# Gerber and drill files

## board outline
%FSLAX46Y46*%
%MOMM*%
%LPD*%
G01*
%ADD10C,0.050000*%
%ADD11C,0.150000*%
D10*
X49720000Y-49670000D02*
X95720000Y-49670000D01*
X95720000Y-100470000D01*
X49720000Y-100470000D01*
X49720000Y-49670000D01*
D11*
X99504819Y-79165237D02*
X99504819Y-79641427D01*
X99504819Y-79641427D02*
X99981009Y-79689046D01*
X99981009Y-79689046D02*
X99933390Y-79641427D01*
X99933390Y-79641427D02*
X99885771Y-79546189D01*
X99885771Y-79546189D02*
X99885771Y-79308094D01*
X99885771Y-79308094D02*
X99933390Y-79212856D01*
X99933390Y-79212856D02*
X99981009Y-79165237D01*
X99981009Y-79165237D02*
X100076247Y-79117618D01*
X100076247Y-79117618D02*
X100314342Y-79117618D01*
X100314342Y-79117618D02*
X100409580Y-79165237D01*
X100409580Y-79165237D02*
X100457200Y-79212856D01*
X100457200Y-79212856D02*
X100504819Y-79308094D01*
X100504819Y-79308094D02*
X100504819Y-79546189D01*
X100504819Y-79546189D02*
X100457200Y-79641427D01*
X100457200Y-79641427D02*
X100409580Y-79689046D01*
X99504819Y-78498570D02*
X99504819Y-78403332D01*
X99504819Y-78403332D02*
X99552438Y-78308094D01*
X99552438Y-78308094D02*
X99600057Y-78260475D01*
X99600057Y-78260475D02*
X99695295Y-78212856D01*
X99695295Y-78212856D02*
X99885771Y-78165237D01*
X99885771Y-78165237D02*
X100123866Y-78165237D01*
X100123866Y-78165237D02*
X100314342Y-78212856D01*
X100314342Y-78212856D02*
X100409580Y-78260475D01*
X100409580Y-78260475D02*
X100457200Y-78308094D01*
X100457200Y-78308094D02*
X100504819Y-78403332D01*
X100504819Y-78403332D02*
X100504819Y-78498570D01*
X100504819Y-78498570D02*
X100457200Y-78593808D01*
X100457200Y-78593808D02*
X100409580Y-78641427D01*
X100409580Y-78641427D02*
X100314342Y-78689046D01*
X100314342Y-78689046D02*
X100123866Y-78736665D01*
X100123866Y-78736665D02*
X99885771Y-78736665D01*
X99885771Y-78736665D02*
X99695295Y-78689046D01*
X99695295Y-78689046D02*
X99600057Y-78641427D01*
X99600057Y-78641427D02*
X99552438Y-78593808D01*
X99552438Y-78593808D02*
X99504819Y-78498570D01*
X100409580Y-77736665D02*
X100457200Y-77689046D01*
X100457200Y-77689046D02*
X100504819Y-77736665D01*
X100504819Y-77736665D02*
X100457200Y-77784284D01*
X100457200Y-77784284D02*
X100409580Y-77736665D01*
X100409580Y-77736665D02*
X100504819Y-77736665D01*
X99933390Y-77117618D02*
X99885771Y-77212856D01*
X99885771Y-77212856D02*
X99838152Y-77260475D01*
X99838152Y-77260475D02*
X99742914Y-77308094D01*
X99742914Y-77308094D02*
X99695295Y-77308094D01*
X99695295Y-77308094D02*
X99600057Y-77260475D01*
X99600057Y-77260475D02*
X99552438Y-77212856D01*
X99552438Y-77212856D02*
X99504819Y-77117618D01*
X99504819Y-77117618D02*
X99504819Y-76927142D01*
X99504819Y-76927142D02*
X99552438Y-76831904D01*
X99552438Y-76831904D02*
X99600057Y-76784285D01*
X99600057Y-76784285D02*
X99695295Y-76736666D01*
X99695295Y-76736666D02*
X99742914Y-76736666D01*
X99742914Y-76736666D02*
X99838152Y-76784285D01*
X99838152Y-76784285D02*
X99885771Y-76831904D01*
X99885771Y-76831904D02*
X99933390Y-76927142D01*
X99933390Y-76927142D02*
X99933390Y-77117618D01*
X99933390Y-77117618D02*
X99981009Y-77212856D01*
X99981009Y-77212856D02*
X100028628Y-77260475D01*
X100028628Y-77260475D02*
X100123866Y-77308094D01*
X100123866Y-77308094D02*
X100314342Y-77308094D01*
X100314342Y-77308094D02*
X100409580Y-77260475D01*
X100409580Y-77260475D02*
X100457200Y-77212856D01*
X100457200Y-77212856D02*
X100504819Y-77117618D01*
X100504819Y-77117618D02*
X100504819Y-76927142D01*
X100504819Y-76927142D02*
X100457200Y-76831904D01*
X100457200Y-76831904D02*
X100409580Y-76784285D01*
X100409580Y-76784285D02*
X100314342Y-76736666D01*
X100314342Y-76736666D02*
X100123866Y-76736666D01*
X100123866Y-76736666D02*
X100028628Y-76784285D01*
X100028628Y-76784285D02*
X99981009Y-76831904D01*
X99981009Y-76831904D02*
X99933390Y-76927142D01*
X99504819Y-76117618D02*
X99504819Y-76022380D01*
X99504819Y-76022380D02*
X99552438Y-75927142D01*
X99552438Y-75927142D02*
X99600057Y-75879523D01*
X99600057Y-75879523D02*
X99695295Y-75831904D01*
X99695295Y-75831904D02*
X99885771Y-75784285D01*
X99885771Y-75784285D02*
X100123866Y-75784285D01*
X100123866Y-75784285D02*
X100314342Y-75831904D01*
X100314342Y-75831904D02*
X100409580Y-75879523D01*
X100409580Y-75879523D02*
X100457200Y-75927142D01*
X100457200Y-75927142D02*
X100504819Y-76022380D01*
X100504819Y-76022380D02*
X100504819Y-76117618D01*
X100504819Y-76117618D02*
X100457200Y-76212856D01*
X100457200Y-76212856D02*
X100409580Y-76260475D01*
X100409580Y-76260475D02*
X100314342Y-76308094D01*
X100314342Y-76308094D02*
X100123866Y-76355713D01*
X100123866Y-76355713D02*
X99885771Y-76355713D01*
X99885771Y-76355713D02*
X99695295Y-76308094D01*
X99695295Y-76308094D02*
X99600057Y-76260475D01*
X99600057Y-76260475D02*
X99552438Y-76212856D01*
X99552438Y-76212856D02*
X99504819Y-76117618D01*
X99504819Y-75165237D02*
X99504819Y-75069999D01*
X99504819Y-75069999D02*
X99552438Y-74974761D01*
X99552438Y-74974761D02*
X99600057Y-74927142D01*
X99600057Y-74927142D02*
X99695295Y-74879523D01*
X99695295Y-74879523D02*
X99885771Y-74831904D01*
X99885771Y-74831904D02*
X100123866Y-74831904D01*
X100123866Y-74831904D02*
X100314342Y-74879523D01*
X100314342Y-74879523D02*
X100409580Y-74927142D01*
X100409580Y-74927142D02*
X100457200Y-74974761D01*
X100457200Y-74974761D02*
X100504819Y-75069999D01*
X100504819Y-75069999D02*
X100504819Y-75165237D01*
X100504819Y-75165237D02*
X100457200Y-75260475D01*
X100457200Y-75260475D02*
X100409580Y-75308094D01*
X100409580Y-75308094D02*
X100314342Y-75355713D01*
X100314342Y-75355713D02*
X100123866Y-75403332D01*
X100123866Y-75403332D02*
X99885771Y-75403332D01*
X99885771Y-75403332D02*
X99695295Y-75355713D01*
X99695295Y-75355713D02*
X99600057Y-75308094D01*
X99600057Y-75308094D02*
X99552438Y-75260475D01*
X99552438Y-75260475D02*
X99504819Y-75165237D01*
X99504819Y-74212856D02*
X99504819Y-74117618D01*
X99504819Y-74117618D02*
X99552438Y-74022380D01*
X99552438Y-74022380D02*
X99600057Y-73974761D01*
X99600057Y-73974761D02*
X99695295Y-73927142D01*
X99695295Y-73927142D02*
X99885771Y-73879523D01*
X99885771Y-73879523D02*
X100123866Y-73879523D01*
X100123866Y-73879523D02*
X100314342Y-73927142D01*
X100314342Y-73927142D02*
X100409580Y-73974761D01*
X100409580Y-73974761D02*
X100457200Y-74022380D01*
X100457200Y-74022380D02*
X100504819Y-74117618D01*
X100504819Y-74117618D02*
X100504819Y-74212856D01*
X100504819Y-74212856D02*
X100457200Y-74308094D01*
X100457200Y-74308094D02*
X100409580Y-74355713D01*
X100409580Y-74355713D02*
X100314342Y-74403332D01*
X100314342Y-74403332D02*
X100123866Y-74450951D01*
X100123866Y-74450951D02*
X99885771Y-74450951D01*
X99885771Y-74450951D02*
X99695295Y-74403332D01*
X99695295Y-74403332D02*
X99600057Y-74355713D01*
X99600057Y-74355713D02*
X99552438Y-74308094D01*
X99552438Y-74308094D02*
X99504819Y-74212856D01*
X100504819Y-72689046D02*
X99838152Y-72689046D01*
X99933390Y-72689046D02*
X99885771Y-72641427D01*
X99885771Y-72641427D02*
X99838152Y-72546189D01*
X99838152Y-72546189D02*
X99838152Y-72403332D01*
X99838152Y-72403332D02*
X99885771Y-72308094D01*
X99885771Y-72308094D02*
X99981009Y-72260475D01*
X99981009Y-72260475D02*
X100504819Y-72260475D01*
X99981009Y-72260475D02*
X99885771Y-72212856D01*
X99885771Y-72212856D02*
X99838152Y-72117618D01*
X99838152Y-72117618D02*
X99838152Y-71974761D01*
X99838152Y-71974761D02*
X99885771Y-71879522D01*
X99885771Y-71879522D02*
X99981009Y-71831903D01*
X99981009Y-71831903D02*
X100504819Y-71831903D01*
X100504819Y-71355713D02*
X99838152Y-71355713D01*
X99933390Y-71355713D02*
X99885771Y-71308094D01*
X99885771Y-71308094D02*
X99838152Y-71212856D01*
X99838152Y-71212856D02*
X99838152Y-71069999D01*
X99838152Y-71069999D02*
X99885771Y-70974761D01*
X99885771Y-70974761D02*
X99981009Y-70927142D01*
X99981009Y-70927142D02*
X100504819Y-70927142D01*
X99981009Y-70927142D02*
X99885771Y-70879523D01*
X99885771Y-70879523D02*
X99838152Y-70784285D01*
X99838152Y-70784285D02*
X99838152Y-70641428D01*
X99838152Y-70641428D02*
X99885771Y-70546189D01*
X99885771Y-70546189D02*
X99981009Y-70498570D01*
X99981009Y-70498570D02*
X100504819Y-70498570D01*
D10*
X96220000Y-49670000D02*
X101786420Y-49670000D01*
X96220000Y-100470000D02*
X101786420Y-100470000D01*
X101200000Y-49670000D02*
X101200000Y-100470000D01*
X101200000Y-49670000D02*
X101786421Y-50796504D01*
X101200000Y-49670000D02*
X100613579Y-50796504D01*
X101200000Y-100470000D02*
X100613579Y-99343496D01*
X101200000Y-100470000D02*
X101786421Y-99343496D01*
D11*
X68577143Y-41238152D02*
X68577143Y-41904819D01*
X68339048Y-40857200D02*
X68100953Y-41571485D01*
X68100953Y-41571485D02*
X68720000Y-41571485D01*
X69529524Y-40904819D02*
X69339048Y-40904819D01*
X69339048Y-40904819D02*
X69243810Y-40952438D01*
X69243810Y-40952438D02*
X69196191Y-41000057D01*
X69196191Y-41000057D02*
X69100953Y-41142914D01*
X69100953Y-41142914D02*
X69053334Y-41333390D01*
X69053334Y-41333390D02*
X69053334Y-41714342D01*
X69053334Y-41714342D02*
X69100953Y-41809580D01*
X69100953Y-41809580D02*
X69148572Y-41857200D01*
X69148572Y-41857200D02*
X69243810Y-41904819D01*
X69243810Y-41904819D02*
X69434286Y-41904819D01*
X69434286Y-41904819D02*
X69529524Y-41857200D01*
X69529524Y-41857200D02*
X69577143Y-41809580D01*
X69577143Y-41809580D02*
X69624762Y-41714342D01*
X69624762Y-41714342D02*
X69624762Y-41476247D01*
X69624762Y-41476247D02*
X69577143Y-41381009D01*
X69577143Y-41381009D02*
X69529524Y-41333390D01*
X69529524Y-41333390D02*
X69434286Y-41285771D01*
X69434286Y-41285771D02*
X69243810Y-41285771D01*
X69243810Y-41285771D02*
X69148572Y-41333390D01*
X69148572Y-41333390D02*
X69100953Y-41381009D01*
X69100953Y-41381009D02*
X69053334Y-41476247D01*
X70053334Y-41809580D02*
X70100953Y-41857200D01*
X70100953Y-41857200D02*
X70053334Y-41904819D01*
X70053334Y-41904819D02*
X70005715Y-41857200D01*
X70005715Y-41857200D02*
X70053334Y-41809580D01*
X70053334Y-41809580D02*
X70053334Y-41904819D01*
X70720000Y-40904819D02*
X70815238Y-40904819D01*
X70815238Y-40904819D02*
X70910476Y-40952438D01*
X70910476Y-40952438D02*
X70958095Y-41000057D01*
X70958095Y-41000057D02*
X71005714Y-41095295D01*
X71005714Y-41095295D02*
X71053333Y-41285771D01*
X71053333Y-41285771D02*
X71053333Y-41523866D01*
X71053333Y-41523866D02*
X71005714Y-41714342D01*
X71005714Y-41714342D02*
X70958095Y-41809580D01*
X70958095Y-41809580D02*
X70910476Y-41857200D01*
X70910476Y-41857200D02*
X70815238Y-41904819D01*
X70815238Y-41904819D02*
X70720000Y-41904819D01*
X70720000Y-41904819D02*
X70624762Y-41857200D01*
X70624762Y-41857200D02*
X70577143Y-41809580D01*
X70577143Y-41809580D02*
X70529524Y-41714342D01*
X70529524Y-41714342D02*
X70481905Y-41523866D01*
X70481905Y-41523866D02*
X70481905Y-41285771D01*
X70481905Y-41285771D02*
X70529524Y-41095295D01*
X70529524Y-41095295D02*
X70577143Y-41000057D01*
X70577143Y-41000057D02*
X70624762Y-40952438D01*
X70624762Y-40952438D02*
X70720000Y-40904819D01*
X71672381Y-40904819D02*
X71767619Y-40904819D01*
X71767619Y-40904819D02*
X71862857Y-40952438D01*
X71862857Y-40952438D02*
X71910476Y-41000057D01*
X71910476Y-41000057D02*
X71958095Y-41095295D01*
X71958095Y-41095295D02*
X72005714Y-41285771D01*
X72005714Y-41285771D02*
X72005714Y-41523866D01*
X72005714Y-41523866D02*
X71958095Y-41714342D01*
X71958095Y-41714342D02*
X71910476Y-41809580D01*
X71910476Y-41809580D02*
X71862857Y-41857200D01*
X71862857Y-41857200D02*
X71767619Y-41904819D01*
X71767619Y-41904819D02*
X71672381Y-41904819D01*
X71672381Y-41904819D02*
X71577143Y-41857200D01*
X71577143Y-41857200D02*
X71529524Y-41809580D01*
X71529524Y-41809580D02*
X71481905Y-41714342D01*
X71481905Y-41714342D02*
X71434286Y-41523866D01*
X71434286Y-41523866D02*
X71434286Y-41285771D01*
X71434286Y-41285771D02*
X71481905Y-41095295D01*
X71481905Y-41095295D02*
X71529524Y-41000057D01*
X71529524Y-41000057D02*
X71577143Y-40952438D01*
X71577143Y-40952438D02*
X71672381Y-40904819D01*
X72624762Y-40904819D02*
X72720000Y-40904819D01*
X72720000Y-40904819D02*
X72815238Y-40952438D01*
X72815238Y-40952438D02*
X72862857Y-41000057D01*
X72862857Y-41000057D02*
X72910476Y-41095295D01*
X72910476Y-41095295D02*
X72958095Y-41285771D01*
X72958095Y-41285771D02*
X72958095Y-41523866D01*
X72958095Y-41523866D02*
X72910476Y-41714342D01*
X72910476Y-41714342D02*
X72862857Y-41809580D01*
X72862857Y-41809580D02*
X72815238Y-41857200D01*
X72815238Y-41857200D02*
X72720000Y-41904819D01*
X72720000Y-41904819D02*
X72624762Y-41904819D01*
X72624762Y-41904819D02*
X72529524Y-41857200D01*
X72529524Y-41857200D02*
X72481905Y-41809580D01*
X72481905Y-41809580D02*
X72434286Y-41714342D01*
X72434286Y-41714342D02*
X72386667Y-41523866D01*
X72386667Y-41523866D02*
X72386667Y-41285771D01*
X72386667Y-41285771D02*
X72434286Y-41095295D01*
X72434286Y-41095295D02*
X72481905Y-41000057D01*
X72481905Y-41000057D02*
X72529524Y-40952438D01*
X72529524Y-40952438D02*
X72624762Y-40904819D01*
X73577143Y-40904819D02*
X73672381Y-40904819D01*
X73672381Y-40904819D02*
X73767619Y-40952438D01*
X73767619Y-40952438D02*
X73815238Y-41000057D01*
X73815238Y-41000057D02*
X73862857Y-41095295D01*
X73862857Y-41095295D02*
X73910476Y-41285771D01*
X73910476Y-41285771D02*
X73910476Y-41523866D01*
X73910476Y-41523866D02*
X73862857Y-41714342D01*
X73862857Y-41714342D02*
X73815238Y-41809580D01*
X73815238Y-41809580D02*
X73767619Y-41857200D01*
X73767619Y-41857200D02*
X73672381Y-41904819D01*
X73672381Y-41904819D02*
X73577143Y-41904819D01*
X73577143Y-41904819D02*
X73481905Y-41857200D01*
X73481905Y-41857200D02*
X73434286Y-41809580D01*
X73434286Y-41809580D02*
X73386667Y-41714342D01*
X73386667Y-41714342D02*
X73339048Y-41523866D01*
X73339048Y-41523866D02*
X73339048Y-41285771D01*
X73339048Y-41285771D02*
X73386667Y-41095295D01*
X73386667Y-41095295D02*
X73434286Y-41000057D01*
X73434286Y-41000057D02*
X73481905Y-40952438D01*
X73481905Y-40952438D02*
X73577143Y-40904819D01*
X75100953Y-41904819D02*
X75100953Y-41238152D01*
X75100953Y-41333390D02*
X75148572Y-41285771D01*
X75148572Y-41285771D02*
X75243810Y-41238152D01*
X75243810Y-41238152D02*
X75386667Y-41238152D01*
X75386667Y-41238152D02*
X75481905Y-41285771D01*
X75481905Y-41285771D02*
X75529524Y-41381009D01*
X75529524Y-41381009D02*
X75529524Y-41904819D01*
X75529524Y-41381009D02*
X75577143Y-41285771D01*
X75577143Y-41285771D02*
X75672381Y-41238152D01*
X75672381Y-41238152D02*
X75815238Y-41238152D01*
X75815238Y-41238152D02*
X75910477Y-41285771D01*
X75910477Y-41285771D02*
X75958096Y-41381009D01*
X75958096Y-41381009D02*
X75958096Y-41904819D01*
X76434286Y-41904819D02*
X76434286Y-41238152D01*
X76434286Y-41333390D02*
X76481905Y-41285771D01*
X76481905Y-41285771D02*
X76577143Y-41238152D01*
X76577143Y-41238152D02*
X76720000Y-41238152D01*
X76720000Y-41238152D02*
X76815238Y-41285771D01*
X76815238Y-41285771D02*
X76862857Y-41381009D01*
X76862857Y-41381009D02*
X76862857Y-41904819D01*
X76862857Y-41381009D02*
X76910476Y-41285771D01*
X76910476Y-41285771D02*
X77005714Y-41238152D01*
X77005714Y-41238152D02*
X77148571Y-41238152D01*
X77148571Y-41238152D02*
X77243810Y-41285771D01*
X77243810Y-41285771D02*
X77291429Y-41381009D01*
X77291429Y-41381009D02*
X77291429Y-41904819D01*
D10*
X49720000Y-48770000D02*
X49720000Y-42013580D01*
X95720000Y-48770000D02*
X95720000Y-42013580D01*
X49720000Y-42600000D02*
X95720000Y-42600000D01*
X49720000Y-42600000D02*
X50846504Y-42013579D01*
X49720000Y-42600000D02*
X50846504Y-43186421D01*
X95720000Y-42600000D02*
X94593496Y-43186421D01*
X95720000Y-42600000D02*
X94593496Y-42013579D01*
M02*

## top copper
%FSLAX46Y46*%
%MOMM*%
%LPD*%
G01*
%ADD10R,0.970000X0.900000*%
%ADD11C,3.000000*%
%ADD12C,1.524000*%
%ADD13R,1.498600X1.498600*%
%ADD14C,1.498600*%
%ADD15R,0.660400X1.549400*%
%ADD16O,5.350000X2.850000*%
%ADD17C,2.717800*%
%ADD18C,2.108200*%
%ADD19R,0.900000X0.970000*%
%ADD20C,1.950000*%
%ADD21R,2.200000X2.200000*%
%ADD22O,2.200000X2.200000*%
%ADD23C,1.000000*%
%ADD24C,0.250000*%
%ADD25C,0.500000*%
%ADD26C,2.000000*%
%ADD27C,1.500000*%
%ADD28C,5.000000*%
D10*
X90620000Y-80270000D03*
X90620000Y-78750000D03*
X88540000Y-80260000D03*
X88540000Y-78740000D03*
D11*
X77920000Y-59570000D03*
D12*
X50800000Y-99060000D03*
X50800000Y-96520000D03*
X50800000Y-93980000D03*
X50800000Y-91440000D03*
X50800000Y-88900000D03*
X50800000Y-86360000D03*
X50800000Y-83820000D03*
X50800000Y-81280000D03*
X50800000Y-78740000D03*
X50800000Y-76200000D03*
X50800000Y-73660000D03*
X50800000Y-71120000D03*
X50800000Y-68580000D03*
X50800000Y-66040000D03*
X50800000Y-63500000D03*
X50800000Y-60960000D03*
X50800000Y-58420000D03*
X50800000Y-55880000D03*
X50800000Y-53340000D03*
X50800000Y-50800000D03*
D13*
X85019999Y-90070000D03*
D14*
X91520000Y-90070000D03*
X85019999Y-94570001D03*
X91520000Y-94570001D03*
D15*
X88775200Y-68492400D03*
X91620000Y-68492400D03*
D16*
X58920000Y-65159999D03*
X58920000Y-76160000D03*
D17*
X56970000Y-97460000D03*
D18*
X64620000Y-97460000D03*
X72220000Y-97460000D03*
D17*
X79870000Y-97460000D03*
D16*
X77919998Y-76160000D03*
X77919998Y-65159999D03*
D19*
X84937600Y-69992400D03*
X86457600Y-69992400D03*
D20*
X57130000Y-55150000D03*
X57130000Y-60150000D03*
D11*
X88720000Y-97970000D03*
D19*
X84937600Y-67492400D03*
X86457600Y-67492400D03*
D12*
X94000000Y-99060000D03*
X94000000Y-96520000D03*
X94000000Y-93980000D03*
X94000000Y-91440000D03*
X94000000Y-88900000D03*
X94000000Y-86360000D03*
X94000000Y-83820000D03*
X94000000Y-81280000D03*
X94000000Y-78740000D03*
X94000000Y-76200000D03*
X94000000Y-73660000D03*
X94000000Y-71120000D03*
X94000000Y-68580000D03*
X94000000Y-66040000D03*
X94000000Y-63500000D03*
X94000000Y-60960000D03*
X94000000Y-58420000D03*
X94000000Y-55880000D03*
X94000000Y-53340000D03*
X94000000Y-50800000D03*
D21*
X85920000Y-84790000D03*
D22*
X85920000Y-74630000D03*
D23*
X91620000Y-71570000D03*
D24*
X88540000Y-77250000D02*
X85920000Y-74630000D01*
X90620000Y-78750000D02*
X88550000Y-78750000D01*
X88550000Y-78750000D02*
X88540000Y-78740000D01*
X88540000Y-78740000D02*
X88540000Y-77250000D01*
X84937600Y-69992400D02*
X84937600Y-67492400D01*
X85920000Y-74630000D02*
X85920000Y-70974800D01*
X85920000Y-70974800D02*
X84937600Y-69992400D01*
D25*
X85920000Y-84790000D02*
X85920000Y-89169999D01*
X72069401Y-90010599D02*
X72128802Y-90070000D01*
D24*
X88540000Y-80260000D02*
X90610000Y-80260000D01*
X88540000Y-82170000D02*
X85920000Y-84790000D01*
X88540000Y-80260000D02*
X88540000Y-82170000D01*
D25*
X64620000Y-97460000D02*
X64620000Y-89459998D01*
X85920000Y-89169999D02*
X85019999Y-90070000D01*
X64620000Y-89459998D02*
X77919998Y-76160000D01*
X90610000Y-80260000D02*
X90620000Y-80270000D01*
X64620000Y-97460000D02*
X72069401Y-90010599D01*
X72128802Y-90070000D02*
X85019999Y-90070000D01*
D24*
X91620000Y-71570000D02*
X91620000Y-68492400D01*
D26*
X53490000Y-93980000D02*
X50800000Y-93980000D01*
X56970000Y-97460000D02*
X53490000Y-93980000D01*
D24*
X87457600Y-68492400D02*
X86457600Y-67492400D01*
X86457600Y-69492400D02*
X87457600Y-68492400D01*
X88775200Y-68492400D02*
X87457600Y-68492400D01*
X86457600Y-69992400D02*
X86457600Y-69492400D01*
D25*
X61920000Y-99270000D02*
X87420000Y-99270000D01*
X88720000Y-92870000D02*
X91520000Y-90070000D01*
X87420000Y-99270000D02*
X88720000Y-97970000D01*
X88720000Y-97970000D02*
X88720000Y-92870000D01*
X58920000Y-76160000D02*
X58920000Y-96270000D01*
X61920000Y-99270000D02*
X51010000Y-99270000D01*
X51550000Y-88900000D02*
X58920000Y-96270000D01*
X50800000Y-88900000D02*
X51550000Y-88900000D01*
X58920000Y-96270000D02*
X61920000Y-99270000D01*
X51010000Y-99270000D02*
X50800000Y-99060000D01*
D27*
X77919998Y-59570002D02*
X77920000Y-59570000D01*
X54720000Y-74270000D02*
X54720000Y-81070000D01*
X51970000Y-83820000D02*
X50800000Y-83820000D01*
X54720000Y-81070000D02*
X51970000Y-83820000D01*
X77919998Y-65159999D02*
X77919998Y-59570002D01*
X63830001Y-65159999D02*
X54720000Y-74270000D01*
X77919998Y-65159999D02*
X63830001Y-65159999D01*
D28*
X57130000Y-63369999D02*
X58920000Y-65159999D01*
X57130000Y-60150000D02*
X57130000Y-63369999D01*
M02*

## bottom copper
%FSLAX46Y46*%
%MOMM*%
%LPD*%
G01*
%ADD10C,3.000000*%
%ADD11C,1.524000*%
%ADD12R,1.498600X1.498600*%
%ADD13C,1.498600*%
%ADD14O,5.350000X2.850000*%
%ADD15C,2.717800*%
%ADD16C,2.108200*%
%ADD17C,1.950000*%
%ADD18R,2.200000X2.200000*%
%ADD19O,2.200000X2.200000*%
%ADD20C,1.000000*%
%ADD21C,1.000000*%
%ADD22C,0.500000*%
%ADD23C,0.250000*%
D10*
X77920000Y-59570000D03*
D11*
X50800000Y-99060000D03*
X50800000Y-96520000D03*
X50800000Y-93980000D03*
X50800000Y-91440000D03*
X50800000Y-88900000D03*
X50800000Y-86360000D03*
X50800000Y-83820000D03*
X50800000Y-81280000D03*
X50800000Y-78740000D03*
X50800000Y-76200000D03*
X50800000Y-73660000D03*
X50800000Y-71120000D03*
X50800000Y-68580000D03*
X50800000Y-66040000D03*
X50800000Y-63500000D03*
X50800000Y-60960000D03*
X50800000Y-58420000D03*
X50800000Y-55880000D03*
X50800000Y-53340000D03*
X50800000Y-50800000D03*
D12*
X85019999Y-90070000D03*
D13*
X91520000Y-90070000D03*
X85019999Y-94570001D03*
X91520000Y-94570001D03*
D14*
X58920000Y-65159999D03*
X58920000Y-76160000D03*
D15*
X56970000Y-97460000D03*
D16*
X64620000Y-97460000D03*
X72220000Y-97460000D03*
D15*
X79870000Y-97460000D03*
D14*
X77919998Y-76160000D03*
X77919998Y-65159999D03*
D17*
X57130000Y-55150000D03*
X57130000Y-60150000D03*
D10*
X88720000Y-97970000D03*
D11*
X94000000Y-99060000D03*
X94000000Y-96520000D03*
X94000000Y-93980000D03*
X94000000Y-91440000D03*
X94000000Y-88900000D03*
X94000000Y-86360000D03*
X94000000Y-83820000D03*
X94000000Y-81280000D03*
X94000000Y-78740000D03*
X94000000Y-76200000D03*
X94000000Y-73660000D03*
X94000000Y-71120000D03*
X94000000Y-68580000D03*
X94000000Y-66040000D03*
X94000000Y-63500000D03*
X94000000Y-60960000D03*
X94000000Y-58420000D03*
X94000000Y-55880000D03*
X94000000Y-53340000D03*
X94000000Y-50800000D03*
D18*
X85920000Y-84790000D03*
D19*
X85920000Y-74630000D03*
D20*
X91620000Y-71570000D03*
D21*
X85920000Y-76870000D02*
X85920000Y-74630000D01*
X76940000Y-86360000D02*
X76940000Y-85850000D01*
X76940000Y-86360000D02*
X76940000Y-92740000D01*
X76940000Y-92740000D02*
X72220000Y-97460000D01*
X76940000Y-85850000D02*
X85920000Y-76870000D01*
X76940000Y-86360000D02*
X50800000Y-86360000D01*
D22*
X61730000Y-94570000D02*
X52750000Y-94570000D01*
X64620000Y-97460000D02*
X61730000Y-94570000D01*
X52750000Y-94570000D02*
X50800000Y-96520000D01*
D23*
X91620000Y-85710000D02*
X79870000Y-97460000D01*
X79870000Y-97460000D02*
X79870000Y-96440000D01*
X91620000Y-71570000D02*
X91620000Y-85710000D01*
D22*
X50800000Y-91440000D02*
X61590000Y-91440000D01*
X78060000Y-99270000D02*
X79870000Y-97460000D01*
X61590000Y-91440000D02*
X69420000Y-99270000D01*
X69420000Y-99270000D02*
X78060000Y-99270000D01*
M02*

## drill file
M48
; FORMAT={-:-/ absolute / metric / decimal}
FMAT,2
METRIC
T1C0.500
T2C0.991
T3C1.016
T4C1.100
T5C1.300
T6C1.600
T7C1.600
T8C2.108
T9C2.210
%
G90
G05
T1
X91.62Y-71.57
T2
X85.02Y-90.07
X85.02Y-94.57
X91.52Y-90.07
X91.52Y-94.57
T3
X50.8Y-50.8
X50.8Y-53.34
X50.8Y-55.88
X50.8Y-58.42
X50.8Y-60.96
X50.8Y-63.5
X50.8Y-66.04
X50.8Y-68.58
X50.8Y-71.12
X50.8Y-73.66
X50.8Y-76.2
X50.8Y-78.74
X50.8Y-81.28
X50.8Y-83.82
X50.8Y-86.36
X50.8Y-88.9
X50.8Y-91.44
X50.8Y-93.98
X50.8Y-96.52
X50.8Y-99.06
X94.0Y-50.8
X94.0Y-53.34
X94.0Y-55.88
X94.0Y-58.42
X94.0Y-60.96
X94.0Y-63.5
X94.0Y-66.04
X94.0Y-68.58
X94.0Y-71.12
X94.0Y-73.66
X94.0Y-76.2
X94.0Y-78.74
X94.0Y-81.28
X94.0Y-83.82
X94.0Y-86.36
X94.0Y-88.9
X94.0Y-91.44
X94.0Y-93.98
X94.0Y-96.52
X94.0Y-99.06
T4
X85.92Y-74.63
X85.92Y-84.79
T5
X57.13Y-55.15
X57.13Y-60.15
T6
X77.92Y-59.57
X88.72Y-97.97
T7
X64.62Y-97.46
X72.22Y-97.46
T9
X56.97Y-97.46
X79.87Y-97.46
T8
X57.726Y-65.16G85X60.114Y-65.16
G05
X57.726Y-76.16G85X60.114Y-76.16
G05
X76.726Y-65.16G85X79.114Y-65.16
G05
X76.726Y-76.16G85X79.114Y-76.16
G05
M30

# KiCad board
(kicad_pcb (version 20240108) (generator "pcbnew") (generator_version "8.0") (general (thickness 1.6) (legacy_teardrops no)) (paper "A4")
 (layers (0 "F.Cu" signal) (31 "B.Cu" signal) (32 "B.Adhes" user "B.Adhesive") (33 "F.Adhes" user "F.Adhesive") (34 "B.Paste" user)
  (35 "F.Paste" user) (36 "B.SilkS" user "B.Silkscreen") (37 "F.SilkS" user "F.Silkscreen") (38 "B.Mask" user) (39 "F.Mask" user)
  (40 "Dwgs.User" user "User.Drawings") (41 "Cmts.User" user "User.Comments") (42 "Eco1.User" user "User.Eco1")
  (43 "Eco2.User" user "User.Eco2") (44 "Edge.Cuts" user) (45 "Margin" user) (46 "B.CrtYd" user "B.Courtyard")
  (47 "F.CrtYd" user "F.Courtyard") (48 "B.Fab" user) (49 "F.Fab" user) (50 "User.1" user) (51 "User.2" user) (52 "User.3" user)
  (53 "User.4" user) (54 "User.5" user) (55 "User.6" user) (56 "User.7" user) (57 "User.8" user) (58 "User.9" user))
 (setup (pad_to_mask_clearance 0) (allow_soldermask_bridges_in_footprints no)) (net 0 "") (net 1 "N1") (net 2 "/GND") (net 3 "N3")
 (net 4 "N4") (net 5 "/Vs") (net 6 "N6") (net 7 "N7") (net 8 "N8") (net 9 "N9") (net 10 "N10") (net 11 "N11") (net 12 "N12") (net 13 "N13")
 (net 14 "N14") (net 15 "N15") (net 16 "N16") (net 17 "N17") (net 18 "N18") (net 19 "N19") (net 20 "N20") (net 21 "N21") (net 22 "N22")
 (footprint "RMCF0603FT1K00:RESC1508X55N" (layer "F.Cu") (at 90.62 79.51 90)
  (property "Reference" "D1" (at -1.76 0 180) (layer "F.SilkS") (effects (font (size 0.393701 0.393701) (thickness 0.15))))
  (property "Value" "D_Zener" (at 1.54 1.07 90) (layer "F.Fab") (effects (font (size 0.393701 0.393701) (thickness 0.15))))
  (pad "1" smd rect (at -0.76 0 90) (size 0.9 0.97) (layers "F.Cu" "F.Paste" "F.Mask") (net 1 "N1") (solder_mask_margin 0.102))
  (pad "2" smd rect (at 0.76 0 90) (size 0.9 0.97) (layers "F.Cu" "F.Paste" "F.Mask") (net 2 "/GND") (solder_mask_margin 0.102)))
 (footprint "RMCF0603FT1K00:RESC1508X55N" (layer "F.Cu") (at 88.54 79.5 90)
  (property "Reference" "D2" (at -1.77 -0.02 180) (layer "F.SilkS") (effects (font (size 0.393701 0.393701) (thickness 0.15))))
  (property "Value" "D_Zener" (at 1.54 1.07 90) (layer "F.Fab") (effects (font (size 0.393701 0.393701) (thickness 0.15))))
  (pad "1" smd rect (at -0.76 0 90) (size 0.9 0.97) (layers "F.Cu" "F.Paste" "F.Mask") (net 1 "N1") (solder_mask_margin 0.102))
  (pad "2" smd rect (at 0.76 0 90) (size 0.9 0.97) (layers "F.Cu" "F.Paste" "F.Mask") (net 2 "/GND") (solder_mask_margin 0.102)))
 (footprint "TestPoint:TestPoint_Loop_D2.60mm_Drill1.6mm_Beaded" (layer "F.Cu") (at 77.92 59.57)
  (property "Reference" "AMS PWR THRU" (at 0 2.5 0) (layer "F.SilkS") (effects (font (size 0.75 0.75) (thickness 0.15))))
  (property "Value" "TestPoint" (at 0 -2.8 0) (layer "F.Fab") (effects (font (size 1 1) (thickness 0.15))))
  (pad "1" thru_hole circle (at 0 0) (size 3 3) (drill 1.6) (layers "*.Cu" "*.Mask") (remove_unused_layers no) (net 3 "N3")))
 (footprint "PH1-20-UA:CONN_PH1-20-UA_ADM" (layer "F.Cu") (at 50.8 99.06 90)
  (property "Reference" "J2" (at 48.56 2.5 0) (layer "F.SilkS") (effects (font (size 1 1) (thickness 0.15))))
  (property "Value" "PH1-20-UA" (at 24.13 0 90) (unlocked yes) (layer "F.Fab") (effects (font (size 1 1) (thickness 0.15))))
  (pad "1" thru_hole circle (at 0 0 90) (size 1.524 1.524) (drill 1.016) (layers "*.Cu" "*.Mask") (remove_unused_layers no) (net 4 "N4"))
  (pad "2" thru_hole circle (at 2.54 0 90) (size 1.524 1.524) (drill 1.016) (layers "*.Cu" "*.Mask") (remove_unused_layers no) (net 1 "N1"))
  (pad "3" thru_hole circle (at 5.08 0 90) (size 1.524 1.524) (drill 1.016) (layers "*.Cu" "*.Mask") (remove_unused_layers no) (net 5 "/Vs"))
  (pad "4" thru_hole circle (at 7.62 0 90) (size 1.524 1.524) (drill 1.016) (layers "*.Cu" "*.Mask") (remove_unused_layers no) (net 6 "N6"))
  (pad "5" thru_hole circle (at 10.16 0 90) (size 1.524 1.524) (drill 1.016) (layers "*.Cu" "*.Mask") (remove_unused_layers no) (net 4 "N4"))
  (pad "6" thru_hole circle (at 12.7 0 90) (size 1.524 1.524) (drill 1.016) (layers "*.Cu" "*.Mask") (remove_unused_layers no)
   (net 2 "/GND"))
  (pad "7" thru_hole circle (at 15.24 0 90) (size 1.524 1.524) (drill 1.016) (layers "*.Cu" "*.Mask") (remove_unused_layers no) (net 3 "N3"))
  (pad "8" thru_hole circle (at 17.78 0 90) (size 1.524 1.524) (drill 1.016) (layers "*.Cu" "*.Mask") (remove_unused_layers no) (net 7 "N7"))
  (pad "9" thru_hole circle (at 20.32 0 90) (size 1.524 1.524) (drill 1.016) (layers "*.Cu" "*.Mask") (remove_unused_layers no) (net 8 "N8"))
  (pad "10" thru_hole circle (at 22.86 0 90) (size 1.524 1.524) (drill 1.016) (layers "*.Cu" "*.Mask") (remove_unused_layers no)
   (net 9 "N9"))
  (pad "11" thru_hole circle (at 25.4 0 90) (size 1.524 1.524) (drill 1.016) (layers "*.Cu" "*.Mask") (remove_unused_layers no)
   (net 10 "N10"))
  (pad "12" thru_hole circle (at 27.94 0 90) (size 1.524 1.524) (drill 1.016) (layers "*.Cu" "*.Mask") (remove_unused_layers no)
   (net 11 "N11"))
  (pad "13" thru_hole circle (at 30.48 0 90) (size 1.524 1.524) (drill 1.016) (layers "*.Cu" "*.Mask") (remove_unused_layers no)
   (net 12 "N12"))
  (pad "14" thru_hole circle (at 33.02 0 90) (size 1.524 1.524) (drill 1.016) (layers "*.Cu" "*.Mask") (remove_unused_layers no)
   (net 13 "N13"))
  (pad "15" thru_hole circle (at 35.56 0 90) (size 1.524 1.524) (drill 1.016) (layers "*.Cu" "*.Mask") (remove_unused_layers no)
   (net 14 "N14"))
  (pad "16" thru_hole circle (at 38.1 0 90) (size 1.524 1.524) (drill 1.016) (layers "*.Cu" "*.Mask") (remove_unused_layers no)
   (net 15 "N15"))
  (pad "17" thru_hole circle (at 40.64 0 90) (size 1.524 1.524) (drill 1.016) (layers "*.Cu" "*.Mask") (remove_unused_layers no)
   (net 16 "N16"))
  (pad "18" thru_hole circle (at 43.18 0 90) (size 1.524 1.524) (drill 1.016) (layers "*.Cu" "*.Mask") (remove_unused_layers no)
   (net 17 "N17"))
  (pad "19" thru_hole circle (at 45.72 0 90) (size 1.524 1.524) (drill 1.016) (layers "*.Cu" "*.Mask") (remove_unused_layers no)
   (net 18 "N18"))
  (pad "20" thru_hole circle (at 48.26 0 90) (size 1.524 1.524) (drill 1.016) (layers "*.Cu" "*.Mask") (remove_unused_layers no)
   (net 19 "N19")))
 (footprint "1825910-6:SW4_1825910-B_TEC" (layer "F.Cu") (at 91.52 94.570001)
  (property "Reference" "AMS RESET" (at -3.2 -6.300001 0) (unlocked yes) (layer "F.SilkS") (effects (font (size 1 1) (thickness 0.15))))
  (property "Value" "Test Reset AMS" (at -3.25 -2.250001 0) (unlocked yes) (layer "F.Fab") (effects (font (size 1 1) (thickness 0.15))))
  (pad "1" thru_hole rect (at -6.500001 -4.500001) (size 1.4986 1.4986) (drill 0.9906) (layers "*.Cu" "*.Mask") (remove_unused_layers no)
   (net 1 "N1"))
  (pad "2" thru_hole circle (at 0 -4.500001) (size 1.4986 1.4986) (drill 0.9906) (layers "*.Cu" "*.Mask") (remove_unused_layers no)
   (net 4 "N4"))
  (pad "3" thru_hole circle (at -6.500001 0) (size 1.4986 1.4986) (drill 0.9906) (layers "*.Cu" "*.Mask") (remove_unused_layers no))
  (pad "4" thru_hole circle (at 0 0) (size 1.4986 1.4986) (drill 0.9906) (layers "*.Cu" "*.Mask") (remove_unused_layers no)))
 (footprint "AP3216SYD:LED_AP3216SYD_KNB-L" (layer "F.Cu") (at 90.1976 68.4924)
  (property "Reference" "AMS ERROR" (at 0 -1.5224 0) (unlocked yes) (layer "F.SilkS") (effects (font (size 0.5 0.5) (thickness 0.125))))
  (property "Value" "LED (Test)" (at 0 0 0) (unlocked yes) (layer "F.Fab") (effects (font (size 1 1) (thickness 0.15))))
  (pad "1" smd rect (at -1.4224 0) (size 0.6604 1.5494) (layers "F.Cu" "F.Paste" "F.Mask") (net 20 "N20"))
  (pad "2" smd rect (at 1.4224 0) (size 0.6604 1.5494) (layers "F.Cu" "F.Paste" "F.Mask") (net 6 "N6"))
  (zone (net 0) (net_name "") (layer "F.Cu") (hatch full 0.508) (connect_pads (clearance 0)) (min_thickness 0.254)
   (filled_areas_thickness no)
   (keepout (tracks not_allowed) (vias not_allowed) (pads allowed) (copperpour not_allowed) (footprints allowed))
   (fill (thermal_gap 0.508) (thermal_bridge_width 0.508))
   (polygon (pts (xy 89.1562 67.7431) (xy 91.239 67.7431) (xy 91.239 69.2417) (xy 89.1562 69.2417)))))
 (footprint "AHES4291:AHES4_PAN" (layer "F.Cu") (at 58.919999 65.159998)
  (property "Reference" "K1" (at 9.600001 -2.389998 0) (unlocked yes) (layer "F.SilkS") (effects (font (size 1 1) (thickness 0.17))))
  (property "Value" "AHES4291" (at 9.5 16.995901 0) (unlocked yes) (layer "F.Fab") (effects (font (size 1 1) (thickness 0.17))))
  (pad "1" thru_hole oval (at 0.000001 0.000001) (size 5.35 2.85) (drill oval 4.4958 2.1082) (layers "*.Cu" "*.Mask")
   (remove_unused_layers no) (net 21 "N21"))
  (pad "2" thru_hole oval (at 0.000001 11.000002) (size 5.35 2.85) (drill oval 4.4958 2.1082) (layers "*.Cu" "*.Mask")
   (remove_unused_layers no) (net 4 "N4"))
  (pad "3" thru_hole circle (at -1.949999 32.300002) (size 2.7178 2.7178) (drill 2.2098) (layers "*.Cu" "*.Mask") (remove_unused_layers no)
   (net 5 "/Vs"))
  (pad "4" thru_hole circle (at 5.700001 32.300002) (size 2.1082 2.1082) (drill 1.6002) (layers "*.Cu" "*.Mask") (remove_unused_layers no)
   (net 1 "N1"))
  (pad "5" thru_hole circle (at 13.300001 32.300002) (size 2.1082 2.1082) (drill 1.6002) (layers "*.Cu" "*.Mask") (remove_unused_layers no)
   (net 2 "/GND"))
  (pad "6" thru_hole circle (at 20.950001 32.300002) (size 2.7178 2.7178) (drill 2.2098) (layers "*.Cu" "*.Mask") (remove_unused_layers no)
   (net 6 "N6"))
  (pad "7" thru_hole oval (at 18.999999 11.000002) (size 5.35 2.85) (drill oval 4.4958 2.1082) (layers "*.Cu" "*.Mask")
   (remove_unused_layers no) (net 1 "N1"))
  (pad "8" thru_hole oval (at 18.999999 0.000001) (size 5.35 2.85) (drill oval 4.4958 2.1082) (layers "*.Cu" "*.Mask")
   (remove_unused_layers no) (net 3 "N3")))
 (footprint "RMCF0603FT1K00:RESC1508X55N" (layer "F.Cu") (at 85.6976 69.9924)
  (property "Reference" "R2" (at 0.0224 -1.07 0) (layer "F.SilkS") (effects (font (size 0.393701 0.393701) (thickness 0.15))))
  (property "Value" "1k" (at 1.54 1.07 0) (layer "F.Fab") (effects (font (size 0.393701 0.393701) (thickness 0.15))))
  (pad "1" smd rect (at -0.76 0) (size 0.9 0.97) (layers "F.Cu" "F.Paste" "F.Mask") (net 2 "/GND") (solder_mask_margin 0.102))
  (pad "2" smd rect (at 0.76 0) (size 0.9 0.97) (layers "F.Cu" "F.Paste" "F.Mask") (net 20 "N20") (solder_mask_margin 0.102)))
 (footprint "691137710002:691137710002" (layer "F.Cu") (at 57.13 57.65 -90)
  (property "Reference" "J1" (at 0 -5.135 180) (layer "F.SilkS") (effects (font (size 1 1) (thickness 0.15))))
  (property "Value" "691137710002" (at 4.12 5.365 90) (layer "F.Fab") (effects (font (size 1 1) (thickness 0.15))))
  (pad "1" thru_hole circle (at -2.5 0 270) (size 1.95 1.95) (drill 1.3) (layers "*.Cu" "*.Mask") (remove_unused_layers no) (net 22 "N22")
   (solder_mask_margin 0.102))
  (pad "2" thru_hole circle (at 2.5 0 270) (size 1.95 1.95) (drill 1.3) (layers "*.Cu" "*.Mask") (remove_unused_layers no) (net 21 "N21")
   (solder_mask_margin 0.102)))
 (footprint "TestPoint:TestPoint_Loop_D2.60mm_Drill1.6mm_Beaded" (layer "F.Cu") (at 88.72 97.97)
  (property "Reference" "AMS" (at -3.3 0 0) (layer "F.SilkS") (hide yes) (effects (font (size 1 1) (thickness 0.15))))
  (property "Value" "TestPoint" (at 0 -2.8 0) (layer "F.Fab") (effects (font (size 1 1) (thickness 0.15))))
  (pad "1" thru_hole circle (at 0 0) (size 3 3) (drill 1.6) (layers "*.Cu" "*.Mask") (remove_unused_layers no) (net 4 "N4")))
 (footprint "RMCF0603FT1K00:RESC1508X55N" (layer "F.Cu") (at 85.6976 67.4924)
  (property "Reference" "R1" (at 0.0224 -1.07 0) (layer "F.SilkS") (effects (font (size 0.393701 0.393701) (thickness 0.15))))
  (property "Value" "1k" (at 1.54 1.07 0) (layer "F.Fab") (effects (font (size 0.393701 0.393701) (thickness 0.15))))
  (pad "1" smd rect (at -0.76 0) (size 0.9 0.97) (layers "F.Cu" "F.Paste" "F.Mask") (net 2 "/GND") (solder_mask_margin 0.102))
  (pad "2" smd rect (at 0.76 0) (size 0.9 0.97) (layers "F.Cu" "F.Paste" "F.Mask") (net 20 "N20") (solder_mask_margin 0.102)))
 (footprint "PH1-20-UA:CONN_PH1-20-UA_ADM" (layer "F.Cu") (at 94 99.06 90)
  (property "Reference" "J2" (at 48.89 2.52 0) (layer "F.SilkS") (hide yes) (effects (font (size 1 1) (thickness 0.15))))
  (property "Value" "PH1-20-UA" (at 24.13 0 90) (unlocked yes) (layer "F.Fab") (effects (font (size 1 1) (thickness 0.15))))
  (pad "1" thru_hole circle (at 0 0 90) (size 1.524 1.524) (drill 1.016) (layers "*.Cu" "*.Mask") (remove_unused_layers no))
  (pad "2" thru_hole circle (at 2.54 0 90) (size 1.524 1.524) (drill 1.016) (layers "*.Cu" "*.Mask") (remove_unused_layers no))
  (pad "3" thru_hole circle (at 5.08 0 90) (size 1.524 1.524) (drill 1.016) (layers "*.Cu" "*.Mask") (remove_unused_layers no))
  (pad "4" thru_hole circle (at 7.62 0 90) (size 1.524 1.524) (drill 1.016) (layers "*.Cu" "*.Mask") (remove_unused_layers no))
  (pad "5" thru_hole circle (at 10.16 0 90) (size 1.524 1.524) (drill 1.016) (layers "*.Cu" "*.Mask") (remove_unused_layers no))
  (pad "6" thru_hole circle (at 12.7 0 90) (size 1.524 1.524) (drill 1.016) (layers "*.Cu" "*.Mask") (remove_unused_layers no))
  (pad "7" thru_hole circle (at 15.24 0 90) (size 1.524 1.524) (drill 1.016) (layers "*.Cu" "*.Mask") (remove_unused_layers no))
  (pad "8" thru_hole circle (at 17.78 0 90) (size 1.524 1.524) (drill 1.016) (layers "*.Cu" "*.Mask") (remove_unused_layers no))
  (pad "9" thru_hole circle (at 20.32 0 90) (size 1.524 1.524) (drill 1.016) (layers "*.Cu" "*.Mask") (remove_unused_layers no))
  (pad "10" thru_hole circle (at 22.86 0 90) (size 1.524 1.524) (drill 1.016) (layers "*.Cu" "*.Mask") (remove_unused_layers no))
  (pad "11" thru_hole circle (at 25.4 0 90) (size 1.524 1.524) (drill 1.016) (layers "*.Cu" "*.Mask") (remove_unused_layers no))
  (pad "12" thru_hole circle (at 27.94 0 90) (size 1.524 1.524) (drill 1.016) (layers "*.Cu" "*.Mask") (remove_unused_layers no))
  (pad "13" thru_hole circle (at 30.48 0 90) (size 1.524 1.524) (drill 1.016) (layers "*.Cu" "*.Mask") (remove_unused_layers no))
  (pad "14" thru_hole circle (at 33.02 0 90) (size 1.524 1.524) (drill 1.016) (layers "*.Cu" "*.Mask") (remove_unused_layers no))
  (pad "15" thru_hole circle (at 35.56 0 90) (size 1.524 1.524) (drill 1.016) (layers "*.Cu" "*.Mask") (remove_unused_layers no))
  (pad "16" thru_hole circle (at 38.1 0 90) (size 1.524 1.524) (drill 1.016) (layers "*.Cu" "*.Mask") (remove_unused_layers no))
  (pad "17" thru_hole circle (at 40.64 0 90) (size 1.524 1.524) (drill 1.016) (layers "*.Cu" "*.Mask") (remove_unused_layers no))
  (pad "18" thru_hole circle (at 43.18 0 90) (size 1.524 1.524) (drill 1.016) (layers "*.Cu" "*.Mask") (remove_unused_layers no))
  (pad "19" thru_hole circle (at 45.72 0 90) (size 1.524 1.524) (drill 1.016) (layers "*.Cu" "*.Mask") (remove_unused_layers no))
  (pad "20" thru_hole circle (at 48.26 0 90) (size 1.524 1.524) (drill 1.016) (layers "*.Cu" "*.Mask") (remove_unused_layers no)))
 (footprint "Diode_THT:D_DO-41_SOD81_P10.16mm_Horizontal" (layer "F.Cu") (at 85.92 84.79 90)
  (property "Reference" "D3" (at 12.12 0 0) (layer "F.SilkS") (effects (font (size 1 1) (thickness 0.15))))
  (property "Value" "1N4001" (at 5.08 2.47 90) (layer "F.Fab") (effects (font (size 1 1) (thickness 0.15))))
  (pad "1" thru_hole rect (at 0 0 90) (size 2.2 2.2) (drill 1.1) (layers "*.Cu" "*.Mask") (remove_unused_layers no) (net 1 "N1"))
  (pad "2" thru_hole oval (at 10.16 0 90) (size 2.2 2.2) (drill 1.1) (layers "*.Cu" "*.Mask") (remove_unused_layers no) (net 2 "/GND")))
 (gr_rect (start 49.72 49.67) (end 95.72 100.47) (stroke (width 0.05) (type default)) (fill none) (layer "Edge.Cuts"))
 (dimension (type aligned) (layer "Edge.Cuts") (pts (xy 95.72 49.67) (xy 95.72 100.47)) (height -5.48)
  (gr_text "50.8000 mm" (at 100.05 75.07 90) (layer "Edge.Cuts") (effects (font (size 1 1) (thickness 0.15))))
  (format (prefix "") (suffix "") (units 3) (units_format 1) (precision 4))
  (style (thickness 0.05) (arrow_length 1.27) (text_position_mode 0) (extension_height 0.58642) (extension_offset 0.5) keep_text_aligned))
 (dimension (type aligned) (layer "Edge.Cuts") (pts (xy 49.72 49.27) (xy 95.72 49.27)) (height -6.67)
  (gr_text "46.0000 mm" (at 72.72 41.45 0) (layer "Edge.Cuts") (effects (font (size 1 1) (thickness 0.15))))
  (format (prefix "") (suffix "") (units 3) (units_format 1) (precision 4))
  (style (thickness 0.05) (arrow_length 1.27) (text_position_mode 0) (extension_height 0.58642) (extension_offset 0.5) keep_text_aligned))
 (segment (start 88.54 77.25) (end 85.92 74.63) (width 0.25) (layer "F.Cu") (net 2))
 (segment (start 90.62 78.75) (end 88.55 78.75) (width 0.25) (layer "F.Cu") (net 2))
 (segment (start 88.55 78.75) (end 88.54 78.74) (width 0.25) (layer "F.Cu") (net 2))
 (segment (start 88.54 78.74) (end 88.54 77.25) (width 0.25) (layer "F.Cu") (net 2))
 (segment (start 84.9376 69.9924) (end 84.9376 67.4924) (width 0.25) (layer "F.Cu") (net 2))
 (segment (start 85.92 74.63) (end 85.92 70.9748) (width 0.25) (layer "F.Cu") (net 2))
 (segment (start 85.92 70.9748) (end 84.9376 69.9924) (width 0.25) (layer "F.Cu") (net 2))
 (segment (start 85.92 76.87) (end 85.92 74.63) (width 1) (layer "B.Cu") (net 2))
 (segment (start 76.94 86.36) (end 76.94 85.85) (width 1) (layer "B.Cu") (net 2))
 (segment (start 76.94 86.36) (end 76.94 92.74) (width 1) (layer "B.Cu") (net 2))
 (segment (start 76.94 92.74) (end 72.22 97.46) (width 1) (layer "B.Cu") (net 2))
 (segment (start 76.94 85.85) (end 85.92 76.87) (width 1) (layer "B.Cu") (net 2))
 (segment (start 76.94 86.36) (end 50.8 86.36) (width 1) (layer "B.Cu") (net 2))
 (segment (start 85.92 84.79) (end 85.92 89.169999) (width 0.5) (layer "F.Cu") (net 1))
 (segment (start 72.069401 90.010599) (end 72.128802 90.07) (width 0.5) (layer "F.Cu") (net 1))
 (segment (start 88.54 80.26) (end 90.61 80.26) (width 0.25) (layer "F.Cu") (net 1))
 (segment (start 88.54 82.17) (end 85.92 84.79) (width 0.25) (layer "F.Cu") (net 1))
 (segment (start 88.54 80.26) (end 88.54 82.17) (width 0.25) (layer "F.Cu") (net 1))
 (segment (start 64.62 97.46) (end 64.62 89.459998) (width 0.5) (layer "F.Cu") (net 1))
 (segment (start 85.92 89.169999) (end 85.019999 90.07) (width 0.5) (layer "F.Cu") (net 1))
 (segment (start 64.62 89.459998) (end 77.919998 76.16) (width 0.5) (layer "F.Cu") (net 1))
 (segment (start 90.61 80.26) (end 90.62 80.27) (width 0.5) (layer "F.Cu") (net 1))
 (segment (start 64.62 97.46) (end 72.069401 90.010599) (width 0.5) (layer "F.Cu") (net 1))
 (segment (start 72.128802 90.07) (end 85.019999 90.07) (width 0.5) (layer "F.Cu") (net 1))
 (segment (start 61.73 94.57) (end 52.75 94.57) (width 0.5) (layer "B.Cu") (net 1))
 (segment (start 64.62 97.46) (end 61.73 94.57) (width 0.5) (layer "B.Cu") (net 1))
 (segment (start 52.75 94.57) (end 50.8 96.52) (width 0.5) (layer "B.Cu") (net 1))
 (segment (start 91.62 71.57) (end 91.62 68.4924) (width 0.25) (layer "F.Cu") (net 6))
 (via (at 91.62 71.57) (size 1) (drill 0.5) (layers "F.Cu" "B.Cu") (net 6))
 (segment (start 91.62 85.71) (end 79.87 97.46) (width 0.25) (layer "B.Cu") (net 6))
 (segment (start 79.87 97.46) (end 79.87 96.44) (width 0.25) (layer "B.Cu") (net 6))
 (segment (start 91.62 71.57) (end 91.62 85.71) (width 0.25) (layer "B.Cu") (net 6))
 (segment (start 50.8 91.44) (end 61.59 91.44) (width 0.5) (layer "B.Cu") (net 6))
 (segment (start 78.06 99.27) (end 79.87 97.46) (width 0.5) (layer "B.Cu") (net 6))
 (segment (start 61.59 91.44) (end 69.42 99.27) (width 0.5) (layer "B.Cu") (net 6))
 (segment (start 69.42 99.27) (end 78.06 99.27) (width 0.5) (layer "B.Cu") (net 6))
 (segment (start 53.49 93.98) (end 50.8 93.98) (width 2) (layer "F.Cu") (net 5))
 (segment (start 56.97 97.46) (end 53.49 93.98) (width 2) (layer "F.Cu") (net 5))
 (segment (start 87.4576 68.4924) (end 86.4576 67.4924) (width 0.25) (layer "F.Cu") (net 20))
 (segment (start 86.4576 69.4924) (end 87.4576 68.4924) (width 0.25) (layer "F.Cu") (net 20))
 (segment (start 88.7752 68.4924) (end 87.4576 68.4924) (width 0.25) (layer "F.Cu") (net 20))
 (segment (start 86.4576 69.9924) (end 86.4576 69.4924) (width 0.25) (layer "F.Cu") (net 20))
 (segment (start 61.92 99.27) (end 87.42 99.27) (width 0.5) (layer "F.Cu") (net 4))
 (segment (start 88.72 92.87) (end 91.52 90.07) (width 0.5) (layer "F.Cu") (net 4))
 (segment (start 87.42 99.27) (end 88.72 97.97) (width 0.5) (layer "F.Cu") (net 4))
 (segment (start 88.72 97.97) (end 88.72 92.87) (width 0.5) (layer "F.Cu") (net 4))
 (segment (start 58.92 76.16) (end 58.92 96.27) (width 0.5) (layer "F.Cu") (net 4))
 (segment (start 61.92 99.27) (end 51.01 99.27) (width 0.5) (layer "F.Cu") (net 4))
 (segment (start 51.55 88.9) (end 58.92 96.27) (width 0.5) (layer "F.Cu") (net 4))
 (segment (start 50.8 88.9) (end 51.55 88.9) (width 0.5) (layer "F.Cu") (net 4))
 (segment (start 58.92 96.27) (end 61.92 99.27) (width 0.5) (layer "F.Cu") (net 4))
 (segment (start 51.01 99.27) (end 50.8 99.06) (width 0.5) (layer "F.Cu") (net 4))
 (segment (start 77.919998 59.570002) (end 77.92 59.57) (width 1.5) (layer "F.Cu") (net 3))
 (segment (start 54.72 74.27) (end 54.72 81.07) (width 1.5) (layer "F.Cu") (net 3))
 (segment (start 51.97 83.82) (end 50.8 83.82) (width 1.5) (layer "F.Cu") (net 3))
 (segment (start 54.72 81.07) (end 51.97 83.82) (width 1.5) (layer "F.Cu") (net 3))
 (segment (start 77.919998 65.159999) (end 77.919998 59.570002) (width 1.5) (layer "F.Cu") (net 3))
 (segment (start 63.830001 65.159999) (end 54.72 74.27) (width 1.5) (layer "F.Cu") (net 3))
 (segment (start 77.919998 65.159999) (end 63.830001 65.159999) (width 1.5) (layer "F.Cu") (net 3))
 (segment (start 57.13 63.369999) (end 58.92 65.159999) (width 5) (layer "F.Cu") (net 21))
 (segment (start 57.13 60.15) (end 57.13 63.369999) (width 5) (layer "F.Cu") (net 21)))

